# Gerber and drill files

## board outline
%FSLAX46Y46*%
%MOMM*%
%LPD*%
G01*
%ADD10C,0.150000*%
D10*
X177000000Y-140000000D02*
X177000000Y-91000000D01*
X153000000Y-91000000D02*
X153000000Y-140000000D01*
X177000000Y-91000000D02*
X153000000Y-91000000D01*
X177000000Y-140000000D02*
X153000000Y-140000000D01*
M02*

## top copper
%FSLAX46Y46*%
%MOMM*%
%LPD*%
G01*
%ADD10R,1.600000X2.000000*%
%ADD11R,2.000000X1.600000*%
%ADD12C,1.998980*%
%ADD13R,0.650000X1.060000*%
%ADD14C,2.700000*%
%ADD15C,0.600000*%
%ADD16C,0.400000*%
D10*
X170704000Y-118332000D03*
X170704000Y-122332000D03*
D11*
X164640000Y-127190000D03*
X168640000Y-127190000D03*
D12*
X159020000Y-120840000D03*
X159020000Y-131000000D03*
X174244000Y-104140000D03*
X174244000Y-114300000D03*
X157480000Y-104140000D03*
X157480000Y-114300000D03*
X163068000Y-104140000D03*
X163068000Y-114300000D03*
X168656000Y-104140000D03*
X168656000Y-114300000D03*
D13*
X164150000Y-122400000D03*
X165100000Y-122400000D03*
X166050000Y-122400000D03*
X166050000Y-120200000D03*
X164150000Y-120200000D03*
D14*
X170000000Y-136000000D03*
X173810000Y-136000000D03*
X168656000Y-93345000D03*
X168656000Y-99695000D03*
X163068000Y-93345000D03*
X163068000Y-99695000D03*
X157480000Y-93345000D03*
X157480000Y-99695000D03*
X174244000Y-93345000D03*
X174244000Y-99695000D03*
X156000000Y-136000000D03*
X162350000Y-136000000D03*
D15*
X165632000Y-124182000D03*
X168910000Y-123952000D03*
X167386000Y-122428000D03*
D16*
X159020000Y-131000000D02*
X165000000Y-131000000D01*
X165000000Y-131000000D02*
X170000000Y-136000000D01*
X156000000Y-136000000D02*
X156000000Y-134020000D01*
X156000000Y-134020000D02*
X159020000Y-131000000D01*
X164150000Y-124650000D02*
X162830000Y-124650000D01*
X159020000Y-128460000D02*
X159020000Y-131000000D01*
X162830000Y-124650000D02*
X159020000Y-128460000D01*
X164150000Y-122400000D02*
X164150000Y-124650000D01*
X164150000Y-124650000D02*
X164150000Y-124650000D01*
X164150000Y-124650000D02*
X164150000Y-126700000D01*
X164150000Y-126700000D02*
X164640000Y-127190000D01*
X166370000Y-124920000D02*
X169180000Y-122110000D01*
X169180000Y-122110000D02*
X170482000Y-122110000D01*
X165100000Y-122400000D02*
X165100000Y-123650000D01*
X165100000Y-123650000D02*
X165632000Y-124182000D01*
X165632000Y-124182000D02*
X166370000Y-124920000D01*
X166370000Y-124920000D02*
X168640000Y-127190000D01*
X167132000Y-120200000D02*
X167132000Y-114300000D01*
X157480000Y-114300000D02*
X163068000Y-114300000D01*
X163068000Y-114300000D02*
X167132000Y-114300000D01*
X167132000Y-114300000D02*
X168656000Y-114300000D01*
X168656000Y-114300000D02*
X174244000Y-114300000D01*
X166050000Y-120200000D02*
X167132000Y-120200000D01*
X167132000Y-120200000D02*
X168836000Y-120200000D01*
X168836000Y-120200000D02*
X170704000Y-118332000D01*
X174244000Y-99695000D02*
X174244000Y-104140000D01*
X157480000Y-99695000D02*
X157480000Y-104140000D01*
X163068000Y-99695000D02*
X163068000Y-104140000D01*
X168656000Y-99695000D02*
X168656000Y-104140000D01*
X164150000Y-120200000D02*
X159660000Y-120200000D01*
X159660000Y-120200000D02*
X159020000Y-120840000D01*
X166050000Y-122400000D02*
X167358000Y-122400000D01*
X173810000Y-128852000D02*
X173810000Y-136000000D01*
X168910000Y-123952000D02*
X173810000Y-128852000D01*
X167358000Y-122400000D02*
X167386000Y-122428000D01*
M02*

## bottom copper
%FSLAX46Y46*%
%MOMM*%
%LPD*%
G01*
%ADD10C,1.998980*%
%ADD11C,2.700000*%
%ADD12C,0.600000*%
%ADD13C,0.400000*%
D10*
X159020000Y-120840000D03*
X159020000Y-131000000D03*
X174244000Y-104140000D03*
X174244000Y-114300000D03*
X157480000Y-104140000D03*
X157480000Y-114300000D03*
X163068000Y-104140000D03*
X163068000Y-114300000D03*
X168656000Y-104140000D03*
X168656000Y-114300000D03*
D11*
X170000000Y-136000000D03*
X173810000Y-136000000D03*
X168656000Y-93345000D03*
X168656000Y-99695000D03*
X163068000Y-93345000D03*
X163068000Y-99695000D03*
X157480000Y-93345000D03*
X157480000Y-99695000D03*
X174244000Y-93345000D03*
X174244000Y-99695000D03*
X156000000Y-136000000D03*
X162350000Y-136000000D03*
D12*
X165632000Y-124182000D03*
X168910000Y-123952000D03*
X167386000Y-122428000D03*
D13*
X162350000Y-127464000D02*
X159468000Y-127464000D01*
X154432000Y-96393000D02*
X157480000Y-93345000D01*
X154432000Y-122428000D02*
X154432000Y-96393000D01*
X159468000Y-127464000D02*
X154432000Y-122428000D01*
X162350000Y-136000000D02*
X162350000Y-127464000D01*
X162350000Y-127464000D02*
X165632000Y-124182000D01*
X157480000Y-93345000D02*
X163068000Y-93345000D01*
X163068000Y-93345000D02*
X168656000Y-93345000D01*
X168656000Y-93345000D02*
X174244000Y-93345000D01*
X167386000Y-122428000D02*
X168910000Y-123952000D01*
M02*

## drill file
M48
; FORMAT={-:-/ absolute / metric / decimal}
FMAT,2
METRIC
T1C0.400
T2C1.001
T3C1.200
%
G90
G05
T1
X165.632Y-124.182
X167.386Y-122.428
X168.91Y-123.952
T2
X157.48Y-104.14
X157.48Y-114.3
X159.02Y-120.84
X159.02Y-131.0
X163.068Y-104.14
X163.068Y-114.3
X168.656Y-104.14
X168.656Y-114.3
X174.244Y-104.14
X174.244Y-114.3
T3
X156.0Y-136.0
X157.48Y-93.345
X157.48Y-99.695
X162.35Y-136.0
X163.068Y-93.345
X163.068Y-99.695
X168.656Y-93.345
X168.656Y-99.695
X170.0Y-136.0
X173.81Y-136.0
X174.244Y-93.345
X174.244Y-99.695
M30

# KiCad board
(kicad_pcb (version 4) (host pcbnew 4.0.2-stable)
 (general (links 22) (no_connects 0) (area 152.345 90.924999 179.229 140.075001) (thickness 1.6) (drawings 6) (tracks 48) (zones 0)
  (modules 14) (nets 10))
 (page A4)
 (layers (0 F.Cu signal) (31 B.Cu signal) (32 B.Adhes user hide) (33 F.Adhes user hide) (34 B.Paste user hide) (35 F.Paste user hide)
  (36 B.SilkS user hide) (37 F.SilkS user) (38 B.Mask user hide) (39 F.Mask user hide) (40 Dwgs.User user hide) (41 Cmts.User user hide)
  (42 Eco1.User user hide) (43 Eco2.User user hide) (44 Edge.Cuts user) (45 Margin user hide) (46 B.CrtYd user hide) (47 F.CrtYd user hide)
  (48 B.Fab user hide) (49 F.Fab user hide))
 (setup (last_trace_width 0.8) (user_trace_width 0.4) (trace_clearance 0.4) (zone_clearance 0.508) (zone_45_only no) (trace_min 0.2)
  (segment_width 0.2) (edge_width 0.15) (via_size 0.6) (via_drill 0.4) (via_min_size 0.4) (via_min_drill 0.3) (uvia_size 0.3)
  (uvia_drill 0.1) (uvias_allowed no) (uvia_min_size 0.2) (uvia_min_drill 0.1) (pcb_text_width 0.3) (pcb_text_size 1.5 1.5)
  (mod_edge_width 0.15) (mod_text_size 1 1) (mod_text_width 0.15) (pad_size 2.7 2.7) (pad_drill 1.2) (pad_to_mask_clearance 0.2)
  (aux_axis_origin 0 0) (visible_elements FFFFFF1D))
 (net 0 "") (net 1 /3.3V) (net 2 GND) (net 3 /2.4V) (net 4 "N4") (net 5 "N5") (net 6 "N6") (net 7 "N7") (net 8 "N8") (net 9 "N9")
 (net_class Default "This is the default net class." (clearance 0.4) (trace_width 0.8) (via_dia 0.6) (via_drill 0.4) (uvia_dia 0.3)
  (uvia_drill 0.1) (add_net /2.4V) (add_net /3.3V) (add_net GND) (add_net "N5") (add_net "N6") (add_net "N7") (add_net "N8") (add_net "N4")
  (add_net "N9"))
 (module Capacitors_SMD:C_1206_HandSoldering (layer F.Cu) (at 170.704 120.332 270)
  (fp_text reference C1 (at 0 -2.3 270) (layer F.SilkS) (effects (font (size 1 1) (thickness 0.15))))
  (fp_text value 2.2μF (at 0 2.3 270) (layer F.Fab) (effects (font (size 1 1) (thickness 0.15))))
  (pad 1 smd rect (at -2 0 270) (size 2 1.6) (layers F.Cu F.Paste F.Mask) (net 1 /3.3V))
  (pad 2 smd rect (at 2 0 270) (size 2 1.6) (layers F.Cu F.Paste F.Mask) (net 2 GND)))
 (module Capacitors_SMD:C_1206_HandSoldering (layer F.Cu) (at 166.64 127.19)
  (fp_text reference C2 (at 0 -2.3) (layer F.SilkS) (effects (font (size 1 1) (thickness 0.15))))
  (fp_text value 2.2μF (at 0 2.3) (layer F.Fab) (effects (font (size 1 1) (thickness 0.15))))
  (pad 1 smd rect (at -2 0) (size 2 1.6) (layers F.Cu F.Paste F.Mask) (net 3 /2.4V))
  (pad 2 smd rect (at 2 0) (size 2 1.6) (layers F.Cu F.Paste F.Mask) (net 2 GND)))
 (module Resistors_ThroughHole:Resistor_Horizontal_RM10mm (layer F.Cu) (at 159.02 120.84 270)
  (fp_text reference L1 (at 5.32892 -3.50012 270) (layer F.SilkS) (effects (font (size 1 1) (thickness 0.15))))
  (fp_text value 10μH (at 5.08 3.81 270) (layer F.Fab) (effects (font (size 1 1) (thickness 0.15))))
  (pad 1 thru_hole circle (at 0 0 270) (size 1.99898 1.99898) (drill 1.00076) (layers *.Cu *.SilkS *.Mask) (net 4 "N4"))
  (pad 2 thru_hole circle (at 10.16 0 270) (size 1.99898 1.99898) (drill 1.00076) (layers *.Cu *.SilkS *.Mask) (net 3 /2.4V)))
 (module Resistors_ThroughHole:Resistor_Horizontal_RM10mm (layer F.Cu) (at 174.244 104.14 270)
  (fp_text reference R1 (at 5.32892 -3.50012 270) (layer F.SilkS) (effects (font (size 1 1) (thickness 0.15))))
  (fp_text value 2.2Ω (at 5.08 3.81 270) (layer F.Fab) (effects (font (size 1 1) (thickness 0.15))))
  (pad 1 thru_hole circle (at 0 0 270) (size 1.99898 1.99898) (drill 1.00076) (layers *.Cu *.SilkS *.Mask) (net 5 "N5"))
  (pad 2 thru_hole circle (at 10.16 0 270) (size 1.99898 1.99898) (drill 1.00076) (layers *.Cu *.SilkS *.Mask) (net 1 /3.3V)))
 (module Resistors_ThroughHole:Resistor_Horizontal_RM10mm (layer F.Cu) (at 157.48 104.14 270)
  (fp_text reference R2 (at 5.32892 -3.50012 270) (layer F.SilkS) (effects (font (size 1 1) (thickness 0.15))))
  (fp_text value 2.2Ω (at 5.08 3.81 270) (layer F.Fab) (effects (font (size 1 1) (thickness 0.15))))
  (pad 1 thru_hole circle (at 0 0 270) (size 1.99898 1.99898) (drill 1.00076) (layers *.Cu *.SilkS *.Mask) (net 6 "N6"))
  (pad 2 thru_hole circle (at 10.16 0 270) (size 1.99898 1.99898) (drill 1.00076) (layers *.Cu *.SilkS *.Mask) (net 1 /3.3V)))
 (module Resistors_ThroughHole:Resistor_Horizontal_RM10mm (layer F.Cu) (at 163.068 104.14 270)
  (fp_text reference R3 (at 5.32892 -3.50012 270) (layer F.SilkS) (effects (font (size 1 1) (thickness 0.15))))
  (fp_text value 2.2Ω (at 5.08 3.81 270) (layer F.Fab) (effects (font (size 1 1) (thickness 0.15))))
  (pad 1 thru_hole circle (at 0 0 270) (size 1.99898 1.99898) (drill 1.00076) (layers *.Cu *.SilkS *.Mask) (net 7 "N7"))
  (pad 2 thru_hole circle (at 10.16 0 270) (size 1.99898 1.99898) (drill 1.00076) (layers *.Cu *.SilkS *.Mask) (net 1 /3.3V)))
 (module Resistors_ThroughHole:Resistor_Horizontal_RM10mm (layer F.Cu) (at 168.656 104.14 270)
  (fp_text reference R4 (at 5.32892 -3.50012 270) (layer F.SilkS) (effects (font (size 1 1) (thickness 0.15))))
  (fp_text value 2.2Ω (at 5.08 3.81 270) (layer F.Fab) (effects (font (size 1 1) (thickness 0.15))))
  (pad 1 thru_hole circle (at 0 0 270) (size 1.99898 1.99898) (drill 1.00076) (layers *.Cu *.SilkS *.Mask) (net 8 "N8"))
  (pad 2 thru_hole circle (at 10.16 0 270) (size 1.99898 1.99898) (drill 1.00076) (layers *.Cu *.SilkS *.Mask) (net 1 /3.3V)))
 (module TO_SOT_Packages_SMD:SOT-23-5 (layer F.Cu) (at 165.1 121.3 90)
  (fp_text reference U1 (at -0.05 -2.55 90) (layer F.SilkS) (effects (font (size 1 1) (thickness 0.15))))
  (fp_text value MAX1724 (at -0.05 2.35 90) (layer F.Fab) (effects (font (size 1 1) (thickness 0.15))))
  (pad 1 smd rect (at -1.1 -0.95 90) (size 1.06 0.65) (layers F.Cu F.Paste F.Mask) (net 3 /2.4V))
  (pad 2 smd rect (at -1.1 0 90) (size 1.06 0.65) (layers F.Cu F.Paste F.Mask) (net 2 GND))
  (pad 3 smd rect (at -1.1 0.95 90) (size 1.06 0.65) (layers F.Cu F.Paste F.Mask) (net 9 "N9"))
  (pad 4 smd rect (at 1.1 0.95 90) (size 1.06 0.65) (layers F.Cu F.Paste F.Mask) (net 1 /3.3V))
  (pad 5 smd rect (at 1.1 -0.95 90) (size 1.06 0.65) (layers F.Cu F.Paste F.Mask) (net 4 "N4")))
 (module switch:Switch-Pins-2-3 (layer F.Cu) (at 170 136)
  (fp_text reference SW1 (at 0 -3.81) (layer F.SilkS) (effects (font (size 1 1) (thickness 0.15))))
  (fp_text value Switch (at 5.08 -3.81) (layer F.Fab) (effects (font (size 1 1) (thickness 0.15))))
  (pad 2 thru_hole circle (at 0 0) (size 2.7 2.7) (drill 1.2) (layers *.Cu *.Mask F.SilkS) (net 3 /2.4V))
  (pad 3 thru_hole circle (at 3.81 0) (size 2.7 2.7) (drill 1.2) (layers *.Cu *.Mask F.SilkS) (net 9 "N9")))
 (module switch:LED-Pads (layer F.Cu) (at 168.656 96.52 270)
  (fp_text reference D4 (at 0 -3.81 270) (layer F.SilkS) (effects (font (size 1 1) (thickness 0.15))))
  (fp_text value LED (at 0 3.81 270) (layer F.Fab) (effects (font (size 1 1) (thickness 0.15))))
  (pad 1 thru_hole circle (at -3.175 0 270) (size 2.7 2.7) (drill 1.2) (layers *.Cu *.Mask F.SilkS) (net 2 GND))
  (pad 2 thru_hole circle (at 3.175 0 270) (size 2.7 2.7) (drill 1.2) (layers *.Cu *.Mask F.SilkS) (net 8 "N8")))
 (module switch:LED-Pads (layer F.Cu) (at 163.068 96.52 270)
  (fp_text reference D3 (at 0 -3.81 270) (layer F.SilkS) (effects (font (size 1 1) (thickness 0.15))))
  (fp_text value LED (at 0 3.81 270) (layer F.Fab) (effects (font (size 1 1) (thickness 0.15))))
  (pad 1 thru_hole circle (at -3.175 0 270) (size 2.7 2.7) (drill 1.2) (layers *.Cu *.Mask F.SilkS) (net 2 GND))
  (pad 2 thru_hole circle (at 3.175 0 270) (size 2.7 2.7) (drill 1.2) (layers *.Cu *.Mask F.SilkS) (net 7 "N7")))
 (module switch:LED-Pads (layer F.Cu) (at 157.48 96.52 270)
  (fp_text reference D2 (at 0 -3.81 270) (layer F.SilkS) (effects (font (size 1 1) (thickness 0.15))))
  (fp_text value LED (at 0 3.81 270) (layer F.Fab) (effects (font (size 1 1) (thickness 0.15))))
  (pad 1 thru_hole circle (at -3.175 0 270) (size 2.7 2.7) (drill 1.2) (layers *.Cu *.Mask F.SilkS) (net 2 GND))
  (pad 2 thru_hole circle (at 3.175 0 270) (size 2.7 2.7) (drill 1.2) (layers *.Cu *.Mask F.SilkS) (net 6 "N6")))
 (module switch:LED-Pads (layer F.Cu) (at 174.244 96.52 270)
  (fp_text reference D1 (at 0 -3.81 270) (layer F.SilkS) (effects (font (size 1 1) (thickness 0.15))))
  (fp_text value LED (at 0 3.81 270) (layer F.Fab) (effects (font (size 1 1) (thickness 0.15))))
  (pad 1 thru_hole circle (at -3.175 0 270) (size 2.7 2.7) (drill 1.2) (layers *.Cu *.Mask F.SilkS) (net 2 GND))
  (pad 2 thru_hole circle (at 3.175 0 270) (size 2.7 2.7) (drill 1.2) (layers *.Cu *.Mask F.SilkS) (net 5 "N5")))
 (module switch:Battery (layer F.Cu) (at 156 136)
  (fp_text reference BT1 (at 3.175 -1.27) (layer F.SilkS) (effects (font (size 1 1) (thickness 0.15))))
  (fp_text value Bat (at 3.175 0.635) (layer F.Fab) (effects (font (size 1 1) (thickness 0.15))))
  (pad 1 thru_hole circle (at 0 0) (size 2.7 2.7) (drill 1.2) (layers *.Cu *.Mask F.SilkS) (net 3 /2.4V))
  (pad 2 thru_hole circle (at 6.35 0) (size 2.7 2.7) (drill 1.2) (layers *.Cu *.Mask F.SilkS) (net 2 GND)))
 (gr_line (start 177 140) (end 177 91) (angle 90) (layer Edge.Cuts) (width 0.15))
 (gr_line (start 153 91) (end 153 140) (angle 90) (layer Edge.Cuts) (width 0.15))
 (gr_line (start 177 91) (end 153 91) (angle 90) (layer Edge.Cuts) (width 0.15))
 (gr_line (start 177 140) (end 153 140) (angle 90) (layer Edge.Cuts) (width 0.15))
 (segment (start 159.02 131) (end 165 131) (width 0.4) (layer F.Cu) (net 3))
 (segment (start 165 131) (end 170 136) (width 0.4) (layer F.Cu) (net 3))
 (segment (start 156 136) (end 156 134.02) (width 0.4) (layer F.Cu) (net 3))
 (segment (start 156 134.02) (end 159.02 131) (width 0.4) (layer F.Cu) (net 3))
 (segment (start 164.15 124.65) (end 162.83 124.65) (width 0.4) (layer F.Cu) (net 3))
 (segment (start 159.02 128.46) (end 159.02 131) (width 0.4) (layer F.Cu) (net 3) (status 20))
 (segment (start 162.83 124.65) (end 159.02 128.46) (width 0.4) (layer F.Cu) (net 3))
 (segment (start 164.15 122.4) (end 164.15 124.65) (width 0.4) (layer F.Cu) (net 3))
 (segment (start 164.15 124.65) (end 164.15 124.65) (width 0.4) (layer F.Cu) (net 3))
 (segment (start 164.15 124.65) (end 164.15 126.7) (width 0.4) (layer F.Cu) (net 3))
 (segment (start 164.15 126.7) (end 164.64 127.19) (width 0.4) (layer F.Cu) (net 3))
 (segment (start 162.35 127.464) (end 159.468 127.464) (width 0.4) (layer B.Cu) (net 2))
 (segment (start 154.432 96.393) (end 157.48 93.345) (width 0.4) (layer B.Cu) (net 2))
 (segment (start 154.432 122.428) (end 154.432 96.393) (width 0.4) (layer B.Cu) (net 2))
 (segment (start 159.468 127.464) (end 154.432 122.428) (width 0.4) (layer B.Cu) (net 2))
 (via (at 165.632 124.182) (size 0.6) (drill 0.4) (layers F.Cu B.Cu) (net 2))
 (segment (start 162.35 136) (end 162.35 127.464) (width 0.4) (layer B.Cu) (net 2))
 (segment (start 162.35 127.464) (end 165.632 124.182) (width 0.4) (layer B.Cu) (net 2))
 (segment (start 157.48 93.345) (end 163.068 93.345) (width 0.4) (layer B.Cu) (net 2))
 (segment (start 163.068 93.345) (end 168.656 93.345) (width 0.4) (layer B.Cu) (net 2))
 (segment (start 168.656 93.345) (end 174.244 93.345) (width 0.4) (layer B.Cu) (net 2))
 (segment (start 166.37 124.92) (end 169.18 122.11) (width 0.4) (layer F.Cu) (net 2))
 (segment (start 169.18 122.11) (end 170.482 122.11) (width 0.4) (layer F.Cu) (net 2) (status 20))
 (segment (start 165.1 122.4) (end 165.1 123.65) (width 0.4) (layer F.Cu) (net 2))
 (segment (start 165.1 123.65) (end 165.632 124.182) (width 0.4) (layer F.Cu) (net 2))
 (segment (start 165.632 124.182) (end 166.37 124.92) (width 0.4) (layer F.Cu) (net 2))
 (segment (start 166.37 124.92) (end 168.64 127.19) (width 0.4) (layer F.Cu) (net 2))
 (segment (start 167.132 120.2) (end 167.132 114.3) (width 0.4) (layer F.Cu) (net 1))
 (segment (start 157.48 114.3) (end 163.068 114.3) (width 0.4) (layer F.Cu) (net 1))
 (segment (start 163.068 114.3) (end 167.132 114.3) (width 0.4) (layer F.Cu) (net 1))
 (segment (start 167.132 114.3) (end 168.656 114.3) (width 0.4) (layer F.Cu) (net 1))
 (segment (start 168.656 114.3) (end 174.244 114.3) (width 0.4) (layer F.Cu) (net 1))
 (segment (start 166.05 120.2) (end 167.132 120.2) (width 0.4) (layer F.Cu) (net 1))
 (segment (start 167.132 120.2) (end 168.836 120.2) (width 0.4) (layer F.Cu) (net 1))
 (segment (start 168.836 120.2) (end 170.704 118.332) (width 0.4) (layer F.Cu) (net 1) (status 20))
 (segment (start 174.244 99.695) (end 174.244 104.14) (width 0.4) (layer F.Cu) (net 5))
 (segment (start 157.48 99.695) (end 157.48 104.14) (width 0.4) (layer F.Cu) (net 6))
 (segment (start 163.068 99.695) (end 163.068 104.14) (width 0.4) (layer F.Cu) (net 7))
 (segment (start 168.656 99.695) (end 168.656 104.14) (width 0.4) (layer F.Cu) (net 8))
 (segment (start 164.15 120.2) (end 159.66 120.2) (width 0.4) (layer F.Cu) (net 4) (status 20))
 (segment (start 159.66 120.2) (end 159.02 120.84) (width 0.4) (layer F.Cu) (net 4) (status 30))
 (segment (start 166.05 122.4) (end 167.358 122.4) (width 0.4) (layer F.Cu) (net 9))
 (segment (start 173.81 128.852) (end 173.81 136) (width 0.4) (layer F.Cu) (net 9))
 (segment (start 168.91 123.952) (end 173.81 128.852) (width 0.4) (layer F.Cu) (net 9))
 (via (at 168.91 123.952) (size 0.6) (drill 0.4) (layers F.Cu B.Cu) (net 9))
 (segment (start 167.386 122.428) (end 168.91 123.952) (width 0.4) (layer B.Cu) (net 9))
 (via (at 167.386 122.428) (size 0.6) (drill 0.4) (layers F.Cu B.Cu) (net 9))
 (segment (start 167.358 122.4) (end 167.386 122.428) (width 0.4) (layer F.Cu) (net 9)))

